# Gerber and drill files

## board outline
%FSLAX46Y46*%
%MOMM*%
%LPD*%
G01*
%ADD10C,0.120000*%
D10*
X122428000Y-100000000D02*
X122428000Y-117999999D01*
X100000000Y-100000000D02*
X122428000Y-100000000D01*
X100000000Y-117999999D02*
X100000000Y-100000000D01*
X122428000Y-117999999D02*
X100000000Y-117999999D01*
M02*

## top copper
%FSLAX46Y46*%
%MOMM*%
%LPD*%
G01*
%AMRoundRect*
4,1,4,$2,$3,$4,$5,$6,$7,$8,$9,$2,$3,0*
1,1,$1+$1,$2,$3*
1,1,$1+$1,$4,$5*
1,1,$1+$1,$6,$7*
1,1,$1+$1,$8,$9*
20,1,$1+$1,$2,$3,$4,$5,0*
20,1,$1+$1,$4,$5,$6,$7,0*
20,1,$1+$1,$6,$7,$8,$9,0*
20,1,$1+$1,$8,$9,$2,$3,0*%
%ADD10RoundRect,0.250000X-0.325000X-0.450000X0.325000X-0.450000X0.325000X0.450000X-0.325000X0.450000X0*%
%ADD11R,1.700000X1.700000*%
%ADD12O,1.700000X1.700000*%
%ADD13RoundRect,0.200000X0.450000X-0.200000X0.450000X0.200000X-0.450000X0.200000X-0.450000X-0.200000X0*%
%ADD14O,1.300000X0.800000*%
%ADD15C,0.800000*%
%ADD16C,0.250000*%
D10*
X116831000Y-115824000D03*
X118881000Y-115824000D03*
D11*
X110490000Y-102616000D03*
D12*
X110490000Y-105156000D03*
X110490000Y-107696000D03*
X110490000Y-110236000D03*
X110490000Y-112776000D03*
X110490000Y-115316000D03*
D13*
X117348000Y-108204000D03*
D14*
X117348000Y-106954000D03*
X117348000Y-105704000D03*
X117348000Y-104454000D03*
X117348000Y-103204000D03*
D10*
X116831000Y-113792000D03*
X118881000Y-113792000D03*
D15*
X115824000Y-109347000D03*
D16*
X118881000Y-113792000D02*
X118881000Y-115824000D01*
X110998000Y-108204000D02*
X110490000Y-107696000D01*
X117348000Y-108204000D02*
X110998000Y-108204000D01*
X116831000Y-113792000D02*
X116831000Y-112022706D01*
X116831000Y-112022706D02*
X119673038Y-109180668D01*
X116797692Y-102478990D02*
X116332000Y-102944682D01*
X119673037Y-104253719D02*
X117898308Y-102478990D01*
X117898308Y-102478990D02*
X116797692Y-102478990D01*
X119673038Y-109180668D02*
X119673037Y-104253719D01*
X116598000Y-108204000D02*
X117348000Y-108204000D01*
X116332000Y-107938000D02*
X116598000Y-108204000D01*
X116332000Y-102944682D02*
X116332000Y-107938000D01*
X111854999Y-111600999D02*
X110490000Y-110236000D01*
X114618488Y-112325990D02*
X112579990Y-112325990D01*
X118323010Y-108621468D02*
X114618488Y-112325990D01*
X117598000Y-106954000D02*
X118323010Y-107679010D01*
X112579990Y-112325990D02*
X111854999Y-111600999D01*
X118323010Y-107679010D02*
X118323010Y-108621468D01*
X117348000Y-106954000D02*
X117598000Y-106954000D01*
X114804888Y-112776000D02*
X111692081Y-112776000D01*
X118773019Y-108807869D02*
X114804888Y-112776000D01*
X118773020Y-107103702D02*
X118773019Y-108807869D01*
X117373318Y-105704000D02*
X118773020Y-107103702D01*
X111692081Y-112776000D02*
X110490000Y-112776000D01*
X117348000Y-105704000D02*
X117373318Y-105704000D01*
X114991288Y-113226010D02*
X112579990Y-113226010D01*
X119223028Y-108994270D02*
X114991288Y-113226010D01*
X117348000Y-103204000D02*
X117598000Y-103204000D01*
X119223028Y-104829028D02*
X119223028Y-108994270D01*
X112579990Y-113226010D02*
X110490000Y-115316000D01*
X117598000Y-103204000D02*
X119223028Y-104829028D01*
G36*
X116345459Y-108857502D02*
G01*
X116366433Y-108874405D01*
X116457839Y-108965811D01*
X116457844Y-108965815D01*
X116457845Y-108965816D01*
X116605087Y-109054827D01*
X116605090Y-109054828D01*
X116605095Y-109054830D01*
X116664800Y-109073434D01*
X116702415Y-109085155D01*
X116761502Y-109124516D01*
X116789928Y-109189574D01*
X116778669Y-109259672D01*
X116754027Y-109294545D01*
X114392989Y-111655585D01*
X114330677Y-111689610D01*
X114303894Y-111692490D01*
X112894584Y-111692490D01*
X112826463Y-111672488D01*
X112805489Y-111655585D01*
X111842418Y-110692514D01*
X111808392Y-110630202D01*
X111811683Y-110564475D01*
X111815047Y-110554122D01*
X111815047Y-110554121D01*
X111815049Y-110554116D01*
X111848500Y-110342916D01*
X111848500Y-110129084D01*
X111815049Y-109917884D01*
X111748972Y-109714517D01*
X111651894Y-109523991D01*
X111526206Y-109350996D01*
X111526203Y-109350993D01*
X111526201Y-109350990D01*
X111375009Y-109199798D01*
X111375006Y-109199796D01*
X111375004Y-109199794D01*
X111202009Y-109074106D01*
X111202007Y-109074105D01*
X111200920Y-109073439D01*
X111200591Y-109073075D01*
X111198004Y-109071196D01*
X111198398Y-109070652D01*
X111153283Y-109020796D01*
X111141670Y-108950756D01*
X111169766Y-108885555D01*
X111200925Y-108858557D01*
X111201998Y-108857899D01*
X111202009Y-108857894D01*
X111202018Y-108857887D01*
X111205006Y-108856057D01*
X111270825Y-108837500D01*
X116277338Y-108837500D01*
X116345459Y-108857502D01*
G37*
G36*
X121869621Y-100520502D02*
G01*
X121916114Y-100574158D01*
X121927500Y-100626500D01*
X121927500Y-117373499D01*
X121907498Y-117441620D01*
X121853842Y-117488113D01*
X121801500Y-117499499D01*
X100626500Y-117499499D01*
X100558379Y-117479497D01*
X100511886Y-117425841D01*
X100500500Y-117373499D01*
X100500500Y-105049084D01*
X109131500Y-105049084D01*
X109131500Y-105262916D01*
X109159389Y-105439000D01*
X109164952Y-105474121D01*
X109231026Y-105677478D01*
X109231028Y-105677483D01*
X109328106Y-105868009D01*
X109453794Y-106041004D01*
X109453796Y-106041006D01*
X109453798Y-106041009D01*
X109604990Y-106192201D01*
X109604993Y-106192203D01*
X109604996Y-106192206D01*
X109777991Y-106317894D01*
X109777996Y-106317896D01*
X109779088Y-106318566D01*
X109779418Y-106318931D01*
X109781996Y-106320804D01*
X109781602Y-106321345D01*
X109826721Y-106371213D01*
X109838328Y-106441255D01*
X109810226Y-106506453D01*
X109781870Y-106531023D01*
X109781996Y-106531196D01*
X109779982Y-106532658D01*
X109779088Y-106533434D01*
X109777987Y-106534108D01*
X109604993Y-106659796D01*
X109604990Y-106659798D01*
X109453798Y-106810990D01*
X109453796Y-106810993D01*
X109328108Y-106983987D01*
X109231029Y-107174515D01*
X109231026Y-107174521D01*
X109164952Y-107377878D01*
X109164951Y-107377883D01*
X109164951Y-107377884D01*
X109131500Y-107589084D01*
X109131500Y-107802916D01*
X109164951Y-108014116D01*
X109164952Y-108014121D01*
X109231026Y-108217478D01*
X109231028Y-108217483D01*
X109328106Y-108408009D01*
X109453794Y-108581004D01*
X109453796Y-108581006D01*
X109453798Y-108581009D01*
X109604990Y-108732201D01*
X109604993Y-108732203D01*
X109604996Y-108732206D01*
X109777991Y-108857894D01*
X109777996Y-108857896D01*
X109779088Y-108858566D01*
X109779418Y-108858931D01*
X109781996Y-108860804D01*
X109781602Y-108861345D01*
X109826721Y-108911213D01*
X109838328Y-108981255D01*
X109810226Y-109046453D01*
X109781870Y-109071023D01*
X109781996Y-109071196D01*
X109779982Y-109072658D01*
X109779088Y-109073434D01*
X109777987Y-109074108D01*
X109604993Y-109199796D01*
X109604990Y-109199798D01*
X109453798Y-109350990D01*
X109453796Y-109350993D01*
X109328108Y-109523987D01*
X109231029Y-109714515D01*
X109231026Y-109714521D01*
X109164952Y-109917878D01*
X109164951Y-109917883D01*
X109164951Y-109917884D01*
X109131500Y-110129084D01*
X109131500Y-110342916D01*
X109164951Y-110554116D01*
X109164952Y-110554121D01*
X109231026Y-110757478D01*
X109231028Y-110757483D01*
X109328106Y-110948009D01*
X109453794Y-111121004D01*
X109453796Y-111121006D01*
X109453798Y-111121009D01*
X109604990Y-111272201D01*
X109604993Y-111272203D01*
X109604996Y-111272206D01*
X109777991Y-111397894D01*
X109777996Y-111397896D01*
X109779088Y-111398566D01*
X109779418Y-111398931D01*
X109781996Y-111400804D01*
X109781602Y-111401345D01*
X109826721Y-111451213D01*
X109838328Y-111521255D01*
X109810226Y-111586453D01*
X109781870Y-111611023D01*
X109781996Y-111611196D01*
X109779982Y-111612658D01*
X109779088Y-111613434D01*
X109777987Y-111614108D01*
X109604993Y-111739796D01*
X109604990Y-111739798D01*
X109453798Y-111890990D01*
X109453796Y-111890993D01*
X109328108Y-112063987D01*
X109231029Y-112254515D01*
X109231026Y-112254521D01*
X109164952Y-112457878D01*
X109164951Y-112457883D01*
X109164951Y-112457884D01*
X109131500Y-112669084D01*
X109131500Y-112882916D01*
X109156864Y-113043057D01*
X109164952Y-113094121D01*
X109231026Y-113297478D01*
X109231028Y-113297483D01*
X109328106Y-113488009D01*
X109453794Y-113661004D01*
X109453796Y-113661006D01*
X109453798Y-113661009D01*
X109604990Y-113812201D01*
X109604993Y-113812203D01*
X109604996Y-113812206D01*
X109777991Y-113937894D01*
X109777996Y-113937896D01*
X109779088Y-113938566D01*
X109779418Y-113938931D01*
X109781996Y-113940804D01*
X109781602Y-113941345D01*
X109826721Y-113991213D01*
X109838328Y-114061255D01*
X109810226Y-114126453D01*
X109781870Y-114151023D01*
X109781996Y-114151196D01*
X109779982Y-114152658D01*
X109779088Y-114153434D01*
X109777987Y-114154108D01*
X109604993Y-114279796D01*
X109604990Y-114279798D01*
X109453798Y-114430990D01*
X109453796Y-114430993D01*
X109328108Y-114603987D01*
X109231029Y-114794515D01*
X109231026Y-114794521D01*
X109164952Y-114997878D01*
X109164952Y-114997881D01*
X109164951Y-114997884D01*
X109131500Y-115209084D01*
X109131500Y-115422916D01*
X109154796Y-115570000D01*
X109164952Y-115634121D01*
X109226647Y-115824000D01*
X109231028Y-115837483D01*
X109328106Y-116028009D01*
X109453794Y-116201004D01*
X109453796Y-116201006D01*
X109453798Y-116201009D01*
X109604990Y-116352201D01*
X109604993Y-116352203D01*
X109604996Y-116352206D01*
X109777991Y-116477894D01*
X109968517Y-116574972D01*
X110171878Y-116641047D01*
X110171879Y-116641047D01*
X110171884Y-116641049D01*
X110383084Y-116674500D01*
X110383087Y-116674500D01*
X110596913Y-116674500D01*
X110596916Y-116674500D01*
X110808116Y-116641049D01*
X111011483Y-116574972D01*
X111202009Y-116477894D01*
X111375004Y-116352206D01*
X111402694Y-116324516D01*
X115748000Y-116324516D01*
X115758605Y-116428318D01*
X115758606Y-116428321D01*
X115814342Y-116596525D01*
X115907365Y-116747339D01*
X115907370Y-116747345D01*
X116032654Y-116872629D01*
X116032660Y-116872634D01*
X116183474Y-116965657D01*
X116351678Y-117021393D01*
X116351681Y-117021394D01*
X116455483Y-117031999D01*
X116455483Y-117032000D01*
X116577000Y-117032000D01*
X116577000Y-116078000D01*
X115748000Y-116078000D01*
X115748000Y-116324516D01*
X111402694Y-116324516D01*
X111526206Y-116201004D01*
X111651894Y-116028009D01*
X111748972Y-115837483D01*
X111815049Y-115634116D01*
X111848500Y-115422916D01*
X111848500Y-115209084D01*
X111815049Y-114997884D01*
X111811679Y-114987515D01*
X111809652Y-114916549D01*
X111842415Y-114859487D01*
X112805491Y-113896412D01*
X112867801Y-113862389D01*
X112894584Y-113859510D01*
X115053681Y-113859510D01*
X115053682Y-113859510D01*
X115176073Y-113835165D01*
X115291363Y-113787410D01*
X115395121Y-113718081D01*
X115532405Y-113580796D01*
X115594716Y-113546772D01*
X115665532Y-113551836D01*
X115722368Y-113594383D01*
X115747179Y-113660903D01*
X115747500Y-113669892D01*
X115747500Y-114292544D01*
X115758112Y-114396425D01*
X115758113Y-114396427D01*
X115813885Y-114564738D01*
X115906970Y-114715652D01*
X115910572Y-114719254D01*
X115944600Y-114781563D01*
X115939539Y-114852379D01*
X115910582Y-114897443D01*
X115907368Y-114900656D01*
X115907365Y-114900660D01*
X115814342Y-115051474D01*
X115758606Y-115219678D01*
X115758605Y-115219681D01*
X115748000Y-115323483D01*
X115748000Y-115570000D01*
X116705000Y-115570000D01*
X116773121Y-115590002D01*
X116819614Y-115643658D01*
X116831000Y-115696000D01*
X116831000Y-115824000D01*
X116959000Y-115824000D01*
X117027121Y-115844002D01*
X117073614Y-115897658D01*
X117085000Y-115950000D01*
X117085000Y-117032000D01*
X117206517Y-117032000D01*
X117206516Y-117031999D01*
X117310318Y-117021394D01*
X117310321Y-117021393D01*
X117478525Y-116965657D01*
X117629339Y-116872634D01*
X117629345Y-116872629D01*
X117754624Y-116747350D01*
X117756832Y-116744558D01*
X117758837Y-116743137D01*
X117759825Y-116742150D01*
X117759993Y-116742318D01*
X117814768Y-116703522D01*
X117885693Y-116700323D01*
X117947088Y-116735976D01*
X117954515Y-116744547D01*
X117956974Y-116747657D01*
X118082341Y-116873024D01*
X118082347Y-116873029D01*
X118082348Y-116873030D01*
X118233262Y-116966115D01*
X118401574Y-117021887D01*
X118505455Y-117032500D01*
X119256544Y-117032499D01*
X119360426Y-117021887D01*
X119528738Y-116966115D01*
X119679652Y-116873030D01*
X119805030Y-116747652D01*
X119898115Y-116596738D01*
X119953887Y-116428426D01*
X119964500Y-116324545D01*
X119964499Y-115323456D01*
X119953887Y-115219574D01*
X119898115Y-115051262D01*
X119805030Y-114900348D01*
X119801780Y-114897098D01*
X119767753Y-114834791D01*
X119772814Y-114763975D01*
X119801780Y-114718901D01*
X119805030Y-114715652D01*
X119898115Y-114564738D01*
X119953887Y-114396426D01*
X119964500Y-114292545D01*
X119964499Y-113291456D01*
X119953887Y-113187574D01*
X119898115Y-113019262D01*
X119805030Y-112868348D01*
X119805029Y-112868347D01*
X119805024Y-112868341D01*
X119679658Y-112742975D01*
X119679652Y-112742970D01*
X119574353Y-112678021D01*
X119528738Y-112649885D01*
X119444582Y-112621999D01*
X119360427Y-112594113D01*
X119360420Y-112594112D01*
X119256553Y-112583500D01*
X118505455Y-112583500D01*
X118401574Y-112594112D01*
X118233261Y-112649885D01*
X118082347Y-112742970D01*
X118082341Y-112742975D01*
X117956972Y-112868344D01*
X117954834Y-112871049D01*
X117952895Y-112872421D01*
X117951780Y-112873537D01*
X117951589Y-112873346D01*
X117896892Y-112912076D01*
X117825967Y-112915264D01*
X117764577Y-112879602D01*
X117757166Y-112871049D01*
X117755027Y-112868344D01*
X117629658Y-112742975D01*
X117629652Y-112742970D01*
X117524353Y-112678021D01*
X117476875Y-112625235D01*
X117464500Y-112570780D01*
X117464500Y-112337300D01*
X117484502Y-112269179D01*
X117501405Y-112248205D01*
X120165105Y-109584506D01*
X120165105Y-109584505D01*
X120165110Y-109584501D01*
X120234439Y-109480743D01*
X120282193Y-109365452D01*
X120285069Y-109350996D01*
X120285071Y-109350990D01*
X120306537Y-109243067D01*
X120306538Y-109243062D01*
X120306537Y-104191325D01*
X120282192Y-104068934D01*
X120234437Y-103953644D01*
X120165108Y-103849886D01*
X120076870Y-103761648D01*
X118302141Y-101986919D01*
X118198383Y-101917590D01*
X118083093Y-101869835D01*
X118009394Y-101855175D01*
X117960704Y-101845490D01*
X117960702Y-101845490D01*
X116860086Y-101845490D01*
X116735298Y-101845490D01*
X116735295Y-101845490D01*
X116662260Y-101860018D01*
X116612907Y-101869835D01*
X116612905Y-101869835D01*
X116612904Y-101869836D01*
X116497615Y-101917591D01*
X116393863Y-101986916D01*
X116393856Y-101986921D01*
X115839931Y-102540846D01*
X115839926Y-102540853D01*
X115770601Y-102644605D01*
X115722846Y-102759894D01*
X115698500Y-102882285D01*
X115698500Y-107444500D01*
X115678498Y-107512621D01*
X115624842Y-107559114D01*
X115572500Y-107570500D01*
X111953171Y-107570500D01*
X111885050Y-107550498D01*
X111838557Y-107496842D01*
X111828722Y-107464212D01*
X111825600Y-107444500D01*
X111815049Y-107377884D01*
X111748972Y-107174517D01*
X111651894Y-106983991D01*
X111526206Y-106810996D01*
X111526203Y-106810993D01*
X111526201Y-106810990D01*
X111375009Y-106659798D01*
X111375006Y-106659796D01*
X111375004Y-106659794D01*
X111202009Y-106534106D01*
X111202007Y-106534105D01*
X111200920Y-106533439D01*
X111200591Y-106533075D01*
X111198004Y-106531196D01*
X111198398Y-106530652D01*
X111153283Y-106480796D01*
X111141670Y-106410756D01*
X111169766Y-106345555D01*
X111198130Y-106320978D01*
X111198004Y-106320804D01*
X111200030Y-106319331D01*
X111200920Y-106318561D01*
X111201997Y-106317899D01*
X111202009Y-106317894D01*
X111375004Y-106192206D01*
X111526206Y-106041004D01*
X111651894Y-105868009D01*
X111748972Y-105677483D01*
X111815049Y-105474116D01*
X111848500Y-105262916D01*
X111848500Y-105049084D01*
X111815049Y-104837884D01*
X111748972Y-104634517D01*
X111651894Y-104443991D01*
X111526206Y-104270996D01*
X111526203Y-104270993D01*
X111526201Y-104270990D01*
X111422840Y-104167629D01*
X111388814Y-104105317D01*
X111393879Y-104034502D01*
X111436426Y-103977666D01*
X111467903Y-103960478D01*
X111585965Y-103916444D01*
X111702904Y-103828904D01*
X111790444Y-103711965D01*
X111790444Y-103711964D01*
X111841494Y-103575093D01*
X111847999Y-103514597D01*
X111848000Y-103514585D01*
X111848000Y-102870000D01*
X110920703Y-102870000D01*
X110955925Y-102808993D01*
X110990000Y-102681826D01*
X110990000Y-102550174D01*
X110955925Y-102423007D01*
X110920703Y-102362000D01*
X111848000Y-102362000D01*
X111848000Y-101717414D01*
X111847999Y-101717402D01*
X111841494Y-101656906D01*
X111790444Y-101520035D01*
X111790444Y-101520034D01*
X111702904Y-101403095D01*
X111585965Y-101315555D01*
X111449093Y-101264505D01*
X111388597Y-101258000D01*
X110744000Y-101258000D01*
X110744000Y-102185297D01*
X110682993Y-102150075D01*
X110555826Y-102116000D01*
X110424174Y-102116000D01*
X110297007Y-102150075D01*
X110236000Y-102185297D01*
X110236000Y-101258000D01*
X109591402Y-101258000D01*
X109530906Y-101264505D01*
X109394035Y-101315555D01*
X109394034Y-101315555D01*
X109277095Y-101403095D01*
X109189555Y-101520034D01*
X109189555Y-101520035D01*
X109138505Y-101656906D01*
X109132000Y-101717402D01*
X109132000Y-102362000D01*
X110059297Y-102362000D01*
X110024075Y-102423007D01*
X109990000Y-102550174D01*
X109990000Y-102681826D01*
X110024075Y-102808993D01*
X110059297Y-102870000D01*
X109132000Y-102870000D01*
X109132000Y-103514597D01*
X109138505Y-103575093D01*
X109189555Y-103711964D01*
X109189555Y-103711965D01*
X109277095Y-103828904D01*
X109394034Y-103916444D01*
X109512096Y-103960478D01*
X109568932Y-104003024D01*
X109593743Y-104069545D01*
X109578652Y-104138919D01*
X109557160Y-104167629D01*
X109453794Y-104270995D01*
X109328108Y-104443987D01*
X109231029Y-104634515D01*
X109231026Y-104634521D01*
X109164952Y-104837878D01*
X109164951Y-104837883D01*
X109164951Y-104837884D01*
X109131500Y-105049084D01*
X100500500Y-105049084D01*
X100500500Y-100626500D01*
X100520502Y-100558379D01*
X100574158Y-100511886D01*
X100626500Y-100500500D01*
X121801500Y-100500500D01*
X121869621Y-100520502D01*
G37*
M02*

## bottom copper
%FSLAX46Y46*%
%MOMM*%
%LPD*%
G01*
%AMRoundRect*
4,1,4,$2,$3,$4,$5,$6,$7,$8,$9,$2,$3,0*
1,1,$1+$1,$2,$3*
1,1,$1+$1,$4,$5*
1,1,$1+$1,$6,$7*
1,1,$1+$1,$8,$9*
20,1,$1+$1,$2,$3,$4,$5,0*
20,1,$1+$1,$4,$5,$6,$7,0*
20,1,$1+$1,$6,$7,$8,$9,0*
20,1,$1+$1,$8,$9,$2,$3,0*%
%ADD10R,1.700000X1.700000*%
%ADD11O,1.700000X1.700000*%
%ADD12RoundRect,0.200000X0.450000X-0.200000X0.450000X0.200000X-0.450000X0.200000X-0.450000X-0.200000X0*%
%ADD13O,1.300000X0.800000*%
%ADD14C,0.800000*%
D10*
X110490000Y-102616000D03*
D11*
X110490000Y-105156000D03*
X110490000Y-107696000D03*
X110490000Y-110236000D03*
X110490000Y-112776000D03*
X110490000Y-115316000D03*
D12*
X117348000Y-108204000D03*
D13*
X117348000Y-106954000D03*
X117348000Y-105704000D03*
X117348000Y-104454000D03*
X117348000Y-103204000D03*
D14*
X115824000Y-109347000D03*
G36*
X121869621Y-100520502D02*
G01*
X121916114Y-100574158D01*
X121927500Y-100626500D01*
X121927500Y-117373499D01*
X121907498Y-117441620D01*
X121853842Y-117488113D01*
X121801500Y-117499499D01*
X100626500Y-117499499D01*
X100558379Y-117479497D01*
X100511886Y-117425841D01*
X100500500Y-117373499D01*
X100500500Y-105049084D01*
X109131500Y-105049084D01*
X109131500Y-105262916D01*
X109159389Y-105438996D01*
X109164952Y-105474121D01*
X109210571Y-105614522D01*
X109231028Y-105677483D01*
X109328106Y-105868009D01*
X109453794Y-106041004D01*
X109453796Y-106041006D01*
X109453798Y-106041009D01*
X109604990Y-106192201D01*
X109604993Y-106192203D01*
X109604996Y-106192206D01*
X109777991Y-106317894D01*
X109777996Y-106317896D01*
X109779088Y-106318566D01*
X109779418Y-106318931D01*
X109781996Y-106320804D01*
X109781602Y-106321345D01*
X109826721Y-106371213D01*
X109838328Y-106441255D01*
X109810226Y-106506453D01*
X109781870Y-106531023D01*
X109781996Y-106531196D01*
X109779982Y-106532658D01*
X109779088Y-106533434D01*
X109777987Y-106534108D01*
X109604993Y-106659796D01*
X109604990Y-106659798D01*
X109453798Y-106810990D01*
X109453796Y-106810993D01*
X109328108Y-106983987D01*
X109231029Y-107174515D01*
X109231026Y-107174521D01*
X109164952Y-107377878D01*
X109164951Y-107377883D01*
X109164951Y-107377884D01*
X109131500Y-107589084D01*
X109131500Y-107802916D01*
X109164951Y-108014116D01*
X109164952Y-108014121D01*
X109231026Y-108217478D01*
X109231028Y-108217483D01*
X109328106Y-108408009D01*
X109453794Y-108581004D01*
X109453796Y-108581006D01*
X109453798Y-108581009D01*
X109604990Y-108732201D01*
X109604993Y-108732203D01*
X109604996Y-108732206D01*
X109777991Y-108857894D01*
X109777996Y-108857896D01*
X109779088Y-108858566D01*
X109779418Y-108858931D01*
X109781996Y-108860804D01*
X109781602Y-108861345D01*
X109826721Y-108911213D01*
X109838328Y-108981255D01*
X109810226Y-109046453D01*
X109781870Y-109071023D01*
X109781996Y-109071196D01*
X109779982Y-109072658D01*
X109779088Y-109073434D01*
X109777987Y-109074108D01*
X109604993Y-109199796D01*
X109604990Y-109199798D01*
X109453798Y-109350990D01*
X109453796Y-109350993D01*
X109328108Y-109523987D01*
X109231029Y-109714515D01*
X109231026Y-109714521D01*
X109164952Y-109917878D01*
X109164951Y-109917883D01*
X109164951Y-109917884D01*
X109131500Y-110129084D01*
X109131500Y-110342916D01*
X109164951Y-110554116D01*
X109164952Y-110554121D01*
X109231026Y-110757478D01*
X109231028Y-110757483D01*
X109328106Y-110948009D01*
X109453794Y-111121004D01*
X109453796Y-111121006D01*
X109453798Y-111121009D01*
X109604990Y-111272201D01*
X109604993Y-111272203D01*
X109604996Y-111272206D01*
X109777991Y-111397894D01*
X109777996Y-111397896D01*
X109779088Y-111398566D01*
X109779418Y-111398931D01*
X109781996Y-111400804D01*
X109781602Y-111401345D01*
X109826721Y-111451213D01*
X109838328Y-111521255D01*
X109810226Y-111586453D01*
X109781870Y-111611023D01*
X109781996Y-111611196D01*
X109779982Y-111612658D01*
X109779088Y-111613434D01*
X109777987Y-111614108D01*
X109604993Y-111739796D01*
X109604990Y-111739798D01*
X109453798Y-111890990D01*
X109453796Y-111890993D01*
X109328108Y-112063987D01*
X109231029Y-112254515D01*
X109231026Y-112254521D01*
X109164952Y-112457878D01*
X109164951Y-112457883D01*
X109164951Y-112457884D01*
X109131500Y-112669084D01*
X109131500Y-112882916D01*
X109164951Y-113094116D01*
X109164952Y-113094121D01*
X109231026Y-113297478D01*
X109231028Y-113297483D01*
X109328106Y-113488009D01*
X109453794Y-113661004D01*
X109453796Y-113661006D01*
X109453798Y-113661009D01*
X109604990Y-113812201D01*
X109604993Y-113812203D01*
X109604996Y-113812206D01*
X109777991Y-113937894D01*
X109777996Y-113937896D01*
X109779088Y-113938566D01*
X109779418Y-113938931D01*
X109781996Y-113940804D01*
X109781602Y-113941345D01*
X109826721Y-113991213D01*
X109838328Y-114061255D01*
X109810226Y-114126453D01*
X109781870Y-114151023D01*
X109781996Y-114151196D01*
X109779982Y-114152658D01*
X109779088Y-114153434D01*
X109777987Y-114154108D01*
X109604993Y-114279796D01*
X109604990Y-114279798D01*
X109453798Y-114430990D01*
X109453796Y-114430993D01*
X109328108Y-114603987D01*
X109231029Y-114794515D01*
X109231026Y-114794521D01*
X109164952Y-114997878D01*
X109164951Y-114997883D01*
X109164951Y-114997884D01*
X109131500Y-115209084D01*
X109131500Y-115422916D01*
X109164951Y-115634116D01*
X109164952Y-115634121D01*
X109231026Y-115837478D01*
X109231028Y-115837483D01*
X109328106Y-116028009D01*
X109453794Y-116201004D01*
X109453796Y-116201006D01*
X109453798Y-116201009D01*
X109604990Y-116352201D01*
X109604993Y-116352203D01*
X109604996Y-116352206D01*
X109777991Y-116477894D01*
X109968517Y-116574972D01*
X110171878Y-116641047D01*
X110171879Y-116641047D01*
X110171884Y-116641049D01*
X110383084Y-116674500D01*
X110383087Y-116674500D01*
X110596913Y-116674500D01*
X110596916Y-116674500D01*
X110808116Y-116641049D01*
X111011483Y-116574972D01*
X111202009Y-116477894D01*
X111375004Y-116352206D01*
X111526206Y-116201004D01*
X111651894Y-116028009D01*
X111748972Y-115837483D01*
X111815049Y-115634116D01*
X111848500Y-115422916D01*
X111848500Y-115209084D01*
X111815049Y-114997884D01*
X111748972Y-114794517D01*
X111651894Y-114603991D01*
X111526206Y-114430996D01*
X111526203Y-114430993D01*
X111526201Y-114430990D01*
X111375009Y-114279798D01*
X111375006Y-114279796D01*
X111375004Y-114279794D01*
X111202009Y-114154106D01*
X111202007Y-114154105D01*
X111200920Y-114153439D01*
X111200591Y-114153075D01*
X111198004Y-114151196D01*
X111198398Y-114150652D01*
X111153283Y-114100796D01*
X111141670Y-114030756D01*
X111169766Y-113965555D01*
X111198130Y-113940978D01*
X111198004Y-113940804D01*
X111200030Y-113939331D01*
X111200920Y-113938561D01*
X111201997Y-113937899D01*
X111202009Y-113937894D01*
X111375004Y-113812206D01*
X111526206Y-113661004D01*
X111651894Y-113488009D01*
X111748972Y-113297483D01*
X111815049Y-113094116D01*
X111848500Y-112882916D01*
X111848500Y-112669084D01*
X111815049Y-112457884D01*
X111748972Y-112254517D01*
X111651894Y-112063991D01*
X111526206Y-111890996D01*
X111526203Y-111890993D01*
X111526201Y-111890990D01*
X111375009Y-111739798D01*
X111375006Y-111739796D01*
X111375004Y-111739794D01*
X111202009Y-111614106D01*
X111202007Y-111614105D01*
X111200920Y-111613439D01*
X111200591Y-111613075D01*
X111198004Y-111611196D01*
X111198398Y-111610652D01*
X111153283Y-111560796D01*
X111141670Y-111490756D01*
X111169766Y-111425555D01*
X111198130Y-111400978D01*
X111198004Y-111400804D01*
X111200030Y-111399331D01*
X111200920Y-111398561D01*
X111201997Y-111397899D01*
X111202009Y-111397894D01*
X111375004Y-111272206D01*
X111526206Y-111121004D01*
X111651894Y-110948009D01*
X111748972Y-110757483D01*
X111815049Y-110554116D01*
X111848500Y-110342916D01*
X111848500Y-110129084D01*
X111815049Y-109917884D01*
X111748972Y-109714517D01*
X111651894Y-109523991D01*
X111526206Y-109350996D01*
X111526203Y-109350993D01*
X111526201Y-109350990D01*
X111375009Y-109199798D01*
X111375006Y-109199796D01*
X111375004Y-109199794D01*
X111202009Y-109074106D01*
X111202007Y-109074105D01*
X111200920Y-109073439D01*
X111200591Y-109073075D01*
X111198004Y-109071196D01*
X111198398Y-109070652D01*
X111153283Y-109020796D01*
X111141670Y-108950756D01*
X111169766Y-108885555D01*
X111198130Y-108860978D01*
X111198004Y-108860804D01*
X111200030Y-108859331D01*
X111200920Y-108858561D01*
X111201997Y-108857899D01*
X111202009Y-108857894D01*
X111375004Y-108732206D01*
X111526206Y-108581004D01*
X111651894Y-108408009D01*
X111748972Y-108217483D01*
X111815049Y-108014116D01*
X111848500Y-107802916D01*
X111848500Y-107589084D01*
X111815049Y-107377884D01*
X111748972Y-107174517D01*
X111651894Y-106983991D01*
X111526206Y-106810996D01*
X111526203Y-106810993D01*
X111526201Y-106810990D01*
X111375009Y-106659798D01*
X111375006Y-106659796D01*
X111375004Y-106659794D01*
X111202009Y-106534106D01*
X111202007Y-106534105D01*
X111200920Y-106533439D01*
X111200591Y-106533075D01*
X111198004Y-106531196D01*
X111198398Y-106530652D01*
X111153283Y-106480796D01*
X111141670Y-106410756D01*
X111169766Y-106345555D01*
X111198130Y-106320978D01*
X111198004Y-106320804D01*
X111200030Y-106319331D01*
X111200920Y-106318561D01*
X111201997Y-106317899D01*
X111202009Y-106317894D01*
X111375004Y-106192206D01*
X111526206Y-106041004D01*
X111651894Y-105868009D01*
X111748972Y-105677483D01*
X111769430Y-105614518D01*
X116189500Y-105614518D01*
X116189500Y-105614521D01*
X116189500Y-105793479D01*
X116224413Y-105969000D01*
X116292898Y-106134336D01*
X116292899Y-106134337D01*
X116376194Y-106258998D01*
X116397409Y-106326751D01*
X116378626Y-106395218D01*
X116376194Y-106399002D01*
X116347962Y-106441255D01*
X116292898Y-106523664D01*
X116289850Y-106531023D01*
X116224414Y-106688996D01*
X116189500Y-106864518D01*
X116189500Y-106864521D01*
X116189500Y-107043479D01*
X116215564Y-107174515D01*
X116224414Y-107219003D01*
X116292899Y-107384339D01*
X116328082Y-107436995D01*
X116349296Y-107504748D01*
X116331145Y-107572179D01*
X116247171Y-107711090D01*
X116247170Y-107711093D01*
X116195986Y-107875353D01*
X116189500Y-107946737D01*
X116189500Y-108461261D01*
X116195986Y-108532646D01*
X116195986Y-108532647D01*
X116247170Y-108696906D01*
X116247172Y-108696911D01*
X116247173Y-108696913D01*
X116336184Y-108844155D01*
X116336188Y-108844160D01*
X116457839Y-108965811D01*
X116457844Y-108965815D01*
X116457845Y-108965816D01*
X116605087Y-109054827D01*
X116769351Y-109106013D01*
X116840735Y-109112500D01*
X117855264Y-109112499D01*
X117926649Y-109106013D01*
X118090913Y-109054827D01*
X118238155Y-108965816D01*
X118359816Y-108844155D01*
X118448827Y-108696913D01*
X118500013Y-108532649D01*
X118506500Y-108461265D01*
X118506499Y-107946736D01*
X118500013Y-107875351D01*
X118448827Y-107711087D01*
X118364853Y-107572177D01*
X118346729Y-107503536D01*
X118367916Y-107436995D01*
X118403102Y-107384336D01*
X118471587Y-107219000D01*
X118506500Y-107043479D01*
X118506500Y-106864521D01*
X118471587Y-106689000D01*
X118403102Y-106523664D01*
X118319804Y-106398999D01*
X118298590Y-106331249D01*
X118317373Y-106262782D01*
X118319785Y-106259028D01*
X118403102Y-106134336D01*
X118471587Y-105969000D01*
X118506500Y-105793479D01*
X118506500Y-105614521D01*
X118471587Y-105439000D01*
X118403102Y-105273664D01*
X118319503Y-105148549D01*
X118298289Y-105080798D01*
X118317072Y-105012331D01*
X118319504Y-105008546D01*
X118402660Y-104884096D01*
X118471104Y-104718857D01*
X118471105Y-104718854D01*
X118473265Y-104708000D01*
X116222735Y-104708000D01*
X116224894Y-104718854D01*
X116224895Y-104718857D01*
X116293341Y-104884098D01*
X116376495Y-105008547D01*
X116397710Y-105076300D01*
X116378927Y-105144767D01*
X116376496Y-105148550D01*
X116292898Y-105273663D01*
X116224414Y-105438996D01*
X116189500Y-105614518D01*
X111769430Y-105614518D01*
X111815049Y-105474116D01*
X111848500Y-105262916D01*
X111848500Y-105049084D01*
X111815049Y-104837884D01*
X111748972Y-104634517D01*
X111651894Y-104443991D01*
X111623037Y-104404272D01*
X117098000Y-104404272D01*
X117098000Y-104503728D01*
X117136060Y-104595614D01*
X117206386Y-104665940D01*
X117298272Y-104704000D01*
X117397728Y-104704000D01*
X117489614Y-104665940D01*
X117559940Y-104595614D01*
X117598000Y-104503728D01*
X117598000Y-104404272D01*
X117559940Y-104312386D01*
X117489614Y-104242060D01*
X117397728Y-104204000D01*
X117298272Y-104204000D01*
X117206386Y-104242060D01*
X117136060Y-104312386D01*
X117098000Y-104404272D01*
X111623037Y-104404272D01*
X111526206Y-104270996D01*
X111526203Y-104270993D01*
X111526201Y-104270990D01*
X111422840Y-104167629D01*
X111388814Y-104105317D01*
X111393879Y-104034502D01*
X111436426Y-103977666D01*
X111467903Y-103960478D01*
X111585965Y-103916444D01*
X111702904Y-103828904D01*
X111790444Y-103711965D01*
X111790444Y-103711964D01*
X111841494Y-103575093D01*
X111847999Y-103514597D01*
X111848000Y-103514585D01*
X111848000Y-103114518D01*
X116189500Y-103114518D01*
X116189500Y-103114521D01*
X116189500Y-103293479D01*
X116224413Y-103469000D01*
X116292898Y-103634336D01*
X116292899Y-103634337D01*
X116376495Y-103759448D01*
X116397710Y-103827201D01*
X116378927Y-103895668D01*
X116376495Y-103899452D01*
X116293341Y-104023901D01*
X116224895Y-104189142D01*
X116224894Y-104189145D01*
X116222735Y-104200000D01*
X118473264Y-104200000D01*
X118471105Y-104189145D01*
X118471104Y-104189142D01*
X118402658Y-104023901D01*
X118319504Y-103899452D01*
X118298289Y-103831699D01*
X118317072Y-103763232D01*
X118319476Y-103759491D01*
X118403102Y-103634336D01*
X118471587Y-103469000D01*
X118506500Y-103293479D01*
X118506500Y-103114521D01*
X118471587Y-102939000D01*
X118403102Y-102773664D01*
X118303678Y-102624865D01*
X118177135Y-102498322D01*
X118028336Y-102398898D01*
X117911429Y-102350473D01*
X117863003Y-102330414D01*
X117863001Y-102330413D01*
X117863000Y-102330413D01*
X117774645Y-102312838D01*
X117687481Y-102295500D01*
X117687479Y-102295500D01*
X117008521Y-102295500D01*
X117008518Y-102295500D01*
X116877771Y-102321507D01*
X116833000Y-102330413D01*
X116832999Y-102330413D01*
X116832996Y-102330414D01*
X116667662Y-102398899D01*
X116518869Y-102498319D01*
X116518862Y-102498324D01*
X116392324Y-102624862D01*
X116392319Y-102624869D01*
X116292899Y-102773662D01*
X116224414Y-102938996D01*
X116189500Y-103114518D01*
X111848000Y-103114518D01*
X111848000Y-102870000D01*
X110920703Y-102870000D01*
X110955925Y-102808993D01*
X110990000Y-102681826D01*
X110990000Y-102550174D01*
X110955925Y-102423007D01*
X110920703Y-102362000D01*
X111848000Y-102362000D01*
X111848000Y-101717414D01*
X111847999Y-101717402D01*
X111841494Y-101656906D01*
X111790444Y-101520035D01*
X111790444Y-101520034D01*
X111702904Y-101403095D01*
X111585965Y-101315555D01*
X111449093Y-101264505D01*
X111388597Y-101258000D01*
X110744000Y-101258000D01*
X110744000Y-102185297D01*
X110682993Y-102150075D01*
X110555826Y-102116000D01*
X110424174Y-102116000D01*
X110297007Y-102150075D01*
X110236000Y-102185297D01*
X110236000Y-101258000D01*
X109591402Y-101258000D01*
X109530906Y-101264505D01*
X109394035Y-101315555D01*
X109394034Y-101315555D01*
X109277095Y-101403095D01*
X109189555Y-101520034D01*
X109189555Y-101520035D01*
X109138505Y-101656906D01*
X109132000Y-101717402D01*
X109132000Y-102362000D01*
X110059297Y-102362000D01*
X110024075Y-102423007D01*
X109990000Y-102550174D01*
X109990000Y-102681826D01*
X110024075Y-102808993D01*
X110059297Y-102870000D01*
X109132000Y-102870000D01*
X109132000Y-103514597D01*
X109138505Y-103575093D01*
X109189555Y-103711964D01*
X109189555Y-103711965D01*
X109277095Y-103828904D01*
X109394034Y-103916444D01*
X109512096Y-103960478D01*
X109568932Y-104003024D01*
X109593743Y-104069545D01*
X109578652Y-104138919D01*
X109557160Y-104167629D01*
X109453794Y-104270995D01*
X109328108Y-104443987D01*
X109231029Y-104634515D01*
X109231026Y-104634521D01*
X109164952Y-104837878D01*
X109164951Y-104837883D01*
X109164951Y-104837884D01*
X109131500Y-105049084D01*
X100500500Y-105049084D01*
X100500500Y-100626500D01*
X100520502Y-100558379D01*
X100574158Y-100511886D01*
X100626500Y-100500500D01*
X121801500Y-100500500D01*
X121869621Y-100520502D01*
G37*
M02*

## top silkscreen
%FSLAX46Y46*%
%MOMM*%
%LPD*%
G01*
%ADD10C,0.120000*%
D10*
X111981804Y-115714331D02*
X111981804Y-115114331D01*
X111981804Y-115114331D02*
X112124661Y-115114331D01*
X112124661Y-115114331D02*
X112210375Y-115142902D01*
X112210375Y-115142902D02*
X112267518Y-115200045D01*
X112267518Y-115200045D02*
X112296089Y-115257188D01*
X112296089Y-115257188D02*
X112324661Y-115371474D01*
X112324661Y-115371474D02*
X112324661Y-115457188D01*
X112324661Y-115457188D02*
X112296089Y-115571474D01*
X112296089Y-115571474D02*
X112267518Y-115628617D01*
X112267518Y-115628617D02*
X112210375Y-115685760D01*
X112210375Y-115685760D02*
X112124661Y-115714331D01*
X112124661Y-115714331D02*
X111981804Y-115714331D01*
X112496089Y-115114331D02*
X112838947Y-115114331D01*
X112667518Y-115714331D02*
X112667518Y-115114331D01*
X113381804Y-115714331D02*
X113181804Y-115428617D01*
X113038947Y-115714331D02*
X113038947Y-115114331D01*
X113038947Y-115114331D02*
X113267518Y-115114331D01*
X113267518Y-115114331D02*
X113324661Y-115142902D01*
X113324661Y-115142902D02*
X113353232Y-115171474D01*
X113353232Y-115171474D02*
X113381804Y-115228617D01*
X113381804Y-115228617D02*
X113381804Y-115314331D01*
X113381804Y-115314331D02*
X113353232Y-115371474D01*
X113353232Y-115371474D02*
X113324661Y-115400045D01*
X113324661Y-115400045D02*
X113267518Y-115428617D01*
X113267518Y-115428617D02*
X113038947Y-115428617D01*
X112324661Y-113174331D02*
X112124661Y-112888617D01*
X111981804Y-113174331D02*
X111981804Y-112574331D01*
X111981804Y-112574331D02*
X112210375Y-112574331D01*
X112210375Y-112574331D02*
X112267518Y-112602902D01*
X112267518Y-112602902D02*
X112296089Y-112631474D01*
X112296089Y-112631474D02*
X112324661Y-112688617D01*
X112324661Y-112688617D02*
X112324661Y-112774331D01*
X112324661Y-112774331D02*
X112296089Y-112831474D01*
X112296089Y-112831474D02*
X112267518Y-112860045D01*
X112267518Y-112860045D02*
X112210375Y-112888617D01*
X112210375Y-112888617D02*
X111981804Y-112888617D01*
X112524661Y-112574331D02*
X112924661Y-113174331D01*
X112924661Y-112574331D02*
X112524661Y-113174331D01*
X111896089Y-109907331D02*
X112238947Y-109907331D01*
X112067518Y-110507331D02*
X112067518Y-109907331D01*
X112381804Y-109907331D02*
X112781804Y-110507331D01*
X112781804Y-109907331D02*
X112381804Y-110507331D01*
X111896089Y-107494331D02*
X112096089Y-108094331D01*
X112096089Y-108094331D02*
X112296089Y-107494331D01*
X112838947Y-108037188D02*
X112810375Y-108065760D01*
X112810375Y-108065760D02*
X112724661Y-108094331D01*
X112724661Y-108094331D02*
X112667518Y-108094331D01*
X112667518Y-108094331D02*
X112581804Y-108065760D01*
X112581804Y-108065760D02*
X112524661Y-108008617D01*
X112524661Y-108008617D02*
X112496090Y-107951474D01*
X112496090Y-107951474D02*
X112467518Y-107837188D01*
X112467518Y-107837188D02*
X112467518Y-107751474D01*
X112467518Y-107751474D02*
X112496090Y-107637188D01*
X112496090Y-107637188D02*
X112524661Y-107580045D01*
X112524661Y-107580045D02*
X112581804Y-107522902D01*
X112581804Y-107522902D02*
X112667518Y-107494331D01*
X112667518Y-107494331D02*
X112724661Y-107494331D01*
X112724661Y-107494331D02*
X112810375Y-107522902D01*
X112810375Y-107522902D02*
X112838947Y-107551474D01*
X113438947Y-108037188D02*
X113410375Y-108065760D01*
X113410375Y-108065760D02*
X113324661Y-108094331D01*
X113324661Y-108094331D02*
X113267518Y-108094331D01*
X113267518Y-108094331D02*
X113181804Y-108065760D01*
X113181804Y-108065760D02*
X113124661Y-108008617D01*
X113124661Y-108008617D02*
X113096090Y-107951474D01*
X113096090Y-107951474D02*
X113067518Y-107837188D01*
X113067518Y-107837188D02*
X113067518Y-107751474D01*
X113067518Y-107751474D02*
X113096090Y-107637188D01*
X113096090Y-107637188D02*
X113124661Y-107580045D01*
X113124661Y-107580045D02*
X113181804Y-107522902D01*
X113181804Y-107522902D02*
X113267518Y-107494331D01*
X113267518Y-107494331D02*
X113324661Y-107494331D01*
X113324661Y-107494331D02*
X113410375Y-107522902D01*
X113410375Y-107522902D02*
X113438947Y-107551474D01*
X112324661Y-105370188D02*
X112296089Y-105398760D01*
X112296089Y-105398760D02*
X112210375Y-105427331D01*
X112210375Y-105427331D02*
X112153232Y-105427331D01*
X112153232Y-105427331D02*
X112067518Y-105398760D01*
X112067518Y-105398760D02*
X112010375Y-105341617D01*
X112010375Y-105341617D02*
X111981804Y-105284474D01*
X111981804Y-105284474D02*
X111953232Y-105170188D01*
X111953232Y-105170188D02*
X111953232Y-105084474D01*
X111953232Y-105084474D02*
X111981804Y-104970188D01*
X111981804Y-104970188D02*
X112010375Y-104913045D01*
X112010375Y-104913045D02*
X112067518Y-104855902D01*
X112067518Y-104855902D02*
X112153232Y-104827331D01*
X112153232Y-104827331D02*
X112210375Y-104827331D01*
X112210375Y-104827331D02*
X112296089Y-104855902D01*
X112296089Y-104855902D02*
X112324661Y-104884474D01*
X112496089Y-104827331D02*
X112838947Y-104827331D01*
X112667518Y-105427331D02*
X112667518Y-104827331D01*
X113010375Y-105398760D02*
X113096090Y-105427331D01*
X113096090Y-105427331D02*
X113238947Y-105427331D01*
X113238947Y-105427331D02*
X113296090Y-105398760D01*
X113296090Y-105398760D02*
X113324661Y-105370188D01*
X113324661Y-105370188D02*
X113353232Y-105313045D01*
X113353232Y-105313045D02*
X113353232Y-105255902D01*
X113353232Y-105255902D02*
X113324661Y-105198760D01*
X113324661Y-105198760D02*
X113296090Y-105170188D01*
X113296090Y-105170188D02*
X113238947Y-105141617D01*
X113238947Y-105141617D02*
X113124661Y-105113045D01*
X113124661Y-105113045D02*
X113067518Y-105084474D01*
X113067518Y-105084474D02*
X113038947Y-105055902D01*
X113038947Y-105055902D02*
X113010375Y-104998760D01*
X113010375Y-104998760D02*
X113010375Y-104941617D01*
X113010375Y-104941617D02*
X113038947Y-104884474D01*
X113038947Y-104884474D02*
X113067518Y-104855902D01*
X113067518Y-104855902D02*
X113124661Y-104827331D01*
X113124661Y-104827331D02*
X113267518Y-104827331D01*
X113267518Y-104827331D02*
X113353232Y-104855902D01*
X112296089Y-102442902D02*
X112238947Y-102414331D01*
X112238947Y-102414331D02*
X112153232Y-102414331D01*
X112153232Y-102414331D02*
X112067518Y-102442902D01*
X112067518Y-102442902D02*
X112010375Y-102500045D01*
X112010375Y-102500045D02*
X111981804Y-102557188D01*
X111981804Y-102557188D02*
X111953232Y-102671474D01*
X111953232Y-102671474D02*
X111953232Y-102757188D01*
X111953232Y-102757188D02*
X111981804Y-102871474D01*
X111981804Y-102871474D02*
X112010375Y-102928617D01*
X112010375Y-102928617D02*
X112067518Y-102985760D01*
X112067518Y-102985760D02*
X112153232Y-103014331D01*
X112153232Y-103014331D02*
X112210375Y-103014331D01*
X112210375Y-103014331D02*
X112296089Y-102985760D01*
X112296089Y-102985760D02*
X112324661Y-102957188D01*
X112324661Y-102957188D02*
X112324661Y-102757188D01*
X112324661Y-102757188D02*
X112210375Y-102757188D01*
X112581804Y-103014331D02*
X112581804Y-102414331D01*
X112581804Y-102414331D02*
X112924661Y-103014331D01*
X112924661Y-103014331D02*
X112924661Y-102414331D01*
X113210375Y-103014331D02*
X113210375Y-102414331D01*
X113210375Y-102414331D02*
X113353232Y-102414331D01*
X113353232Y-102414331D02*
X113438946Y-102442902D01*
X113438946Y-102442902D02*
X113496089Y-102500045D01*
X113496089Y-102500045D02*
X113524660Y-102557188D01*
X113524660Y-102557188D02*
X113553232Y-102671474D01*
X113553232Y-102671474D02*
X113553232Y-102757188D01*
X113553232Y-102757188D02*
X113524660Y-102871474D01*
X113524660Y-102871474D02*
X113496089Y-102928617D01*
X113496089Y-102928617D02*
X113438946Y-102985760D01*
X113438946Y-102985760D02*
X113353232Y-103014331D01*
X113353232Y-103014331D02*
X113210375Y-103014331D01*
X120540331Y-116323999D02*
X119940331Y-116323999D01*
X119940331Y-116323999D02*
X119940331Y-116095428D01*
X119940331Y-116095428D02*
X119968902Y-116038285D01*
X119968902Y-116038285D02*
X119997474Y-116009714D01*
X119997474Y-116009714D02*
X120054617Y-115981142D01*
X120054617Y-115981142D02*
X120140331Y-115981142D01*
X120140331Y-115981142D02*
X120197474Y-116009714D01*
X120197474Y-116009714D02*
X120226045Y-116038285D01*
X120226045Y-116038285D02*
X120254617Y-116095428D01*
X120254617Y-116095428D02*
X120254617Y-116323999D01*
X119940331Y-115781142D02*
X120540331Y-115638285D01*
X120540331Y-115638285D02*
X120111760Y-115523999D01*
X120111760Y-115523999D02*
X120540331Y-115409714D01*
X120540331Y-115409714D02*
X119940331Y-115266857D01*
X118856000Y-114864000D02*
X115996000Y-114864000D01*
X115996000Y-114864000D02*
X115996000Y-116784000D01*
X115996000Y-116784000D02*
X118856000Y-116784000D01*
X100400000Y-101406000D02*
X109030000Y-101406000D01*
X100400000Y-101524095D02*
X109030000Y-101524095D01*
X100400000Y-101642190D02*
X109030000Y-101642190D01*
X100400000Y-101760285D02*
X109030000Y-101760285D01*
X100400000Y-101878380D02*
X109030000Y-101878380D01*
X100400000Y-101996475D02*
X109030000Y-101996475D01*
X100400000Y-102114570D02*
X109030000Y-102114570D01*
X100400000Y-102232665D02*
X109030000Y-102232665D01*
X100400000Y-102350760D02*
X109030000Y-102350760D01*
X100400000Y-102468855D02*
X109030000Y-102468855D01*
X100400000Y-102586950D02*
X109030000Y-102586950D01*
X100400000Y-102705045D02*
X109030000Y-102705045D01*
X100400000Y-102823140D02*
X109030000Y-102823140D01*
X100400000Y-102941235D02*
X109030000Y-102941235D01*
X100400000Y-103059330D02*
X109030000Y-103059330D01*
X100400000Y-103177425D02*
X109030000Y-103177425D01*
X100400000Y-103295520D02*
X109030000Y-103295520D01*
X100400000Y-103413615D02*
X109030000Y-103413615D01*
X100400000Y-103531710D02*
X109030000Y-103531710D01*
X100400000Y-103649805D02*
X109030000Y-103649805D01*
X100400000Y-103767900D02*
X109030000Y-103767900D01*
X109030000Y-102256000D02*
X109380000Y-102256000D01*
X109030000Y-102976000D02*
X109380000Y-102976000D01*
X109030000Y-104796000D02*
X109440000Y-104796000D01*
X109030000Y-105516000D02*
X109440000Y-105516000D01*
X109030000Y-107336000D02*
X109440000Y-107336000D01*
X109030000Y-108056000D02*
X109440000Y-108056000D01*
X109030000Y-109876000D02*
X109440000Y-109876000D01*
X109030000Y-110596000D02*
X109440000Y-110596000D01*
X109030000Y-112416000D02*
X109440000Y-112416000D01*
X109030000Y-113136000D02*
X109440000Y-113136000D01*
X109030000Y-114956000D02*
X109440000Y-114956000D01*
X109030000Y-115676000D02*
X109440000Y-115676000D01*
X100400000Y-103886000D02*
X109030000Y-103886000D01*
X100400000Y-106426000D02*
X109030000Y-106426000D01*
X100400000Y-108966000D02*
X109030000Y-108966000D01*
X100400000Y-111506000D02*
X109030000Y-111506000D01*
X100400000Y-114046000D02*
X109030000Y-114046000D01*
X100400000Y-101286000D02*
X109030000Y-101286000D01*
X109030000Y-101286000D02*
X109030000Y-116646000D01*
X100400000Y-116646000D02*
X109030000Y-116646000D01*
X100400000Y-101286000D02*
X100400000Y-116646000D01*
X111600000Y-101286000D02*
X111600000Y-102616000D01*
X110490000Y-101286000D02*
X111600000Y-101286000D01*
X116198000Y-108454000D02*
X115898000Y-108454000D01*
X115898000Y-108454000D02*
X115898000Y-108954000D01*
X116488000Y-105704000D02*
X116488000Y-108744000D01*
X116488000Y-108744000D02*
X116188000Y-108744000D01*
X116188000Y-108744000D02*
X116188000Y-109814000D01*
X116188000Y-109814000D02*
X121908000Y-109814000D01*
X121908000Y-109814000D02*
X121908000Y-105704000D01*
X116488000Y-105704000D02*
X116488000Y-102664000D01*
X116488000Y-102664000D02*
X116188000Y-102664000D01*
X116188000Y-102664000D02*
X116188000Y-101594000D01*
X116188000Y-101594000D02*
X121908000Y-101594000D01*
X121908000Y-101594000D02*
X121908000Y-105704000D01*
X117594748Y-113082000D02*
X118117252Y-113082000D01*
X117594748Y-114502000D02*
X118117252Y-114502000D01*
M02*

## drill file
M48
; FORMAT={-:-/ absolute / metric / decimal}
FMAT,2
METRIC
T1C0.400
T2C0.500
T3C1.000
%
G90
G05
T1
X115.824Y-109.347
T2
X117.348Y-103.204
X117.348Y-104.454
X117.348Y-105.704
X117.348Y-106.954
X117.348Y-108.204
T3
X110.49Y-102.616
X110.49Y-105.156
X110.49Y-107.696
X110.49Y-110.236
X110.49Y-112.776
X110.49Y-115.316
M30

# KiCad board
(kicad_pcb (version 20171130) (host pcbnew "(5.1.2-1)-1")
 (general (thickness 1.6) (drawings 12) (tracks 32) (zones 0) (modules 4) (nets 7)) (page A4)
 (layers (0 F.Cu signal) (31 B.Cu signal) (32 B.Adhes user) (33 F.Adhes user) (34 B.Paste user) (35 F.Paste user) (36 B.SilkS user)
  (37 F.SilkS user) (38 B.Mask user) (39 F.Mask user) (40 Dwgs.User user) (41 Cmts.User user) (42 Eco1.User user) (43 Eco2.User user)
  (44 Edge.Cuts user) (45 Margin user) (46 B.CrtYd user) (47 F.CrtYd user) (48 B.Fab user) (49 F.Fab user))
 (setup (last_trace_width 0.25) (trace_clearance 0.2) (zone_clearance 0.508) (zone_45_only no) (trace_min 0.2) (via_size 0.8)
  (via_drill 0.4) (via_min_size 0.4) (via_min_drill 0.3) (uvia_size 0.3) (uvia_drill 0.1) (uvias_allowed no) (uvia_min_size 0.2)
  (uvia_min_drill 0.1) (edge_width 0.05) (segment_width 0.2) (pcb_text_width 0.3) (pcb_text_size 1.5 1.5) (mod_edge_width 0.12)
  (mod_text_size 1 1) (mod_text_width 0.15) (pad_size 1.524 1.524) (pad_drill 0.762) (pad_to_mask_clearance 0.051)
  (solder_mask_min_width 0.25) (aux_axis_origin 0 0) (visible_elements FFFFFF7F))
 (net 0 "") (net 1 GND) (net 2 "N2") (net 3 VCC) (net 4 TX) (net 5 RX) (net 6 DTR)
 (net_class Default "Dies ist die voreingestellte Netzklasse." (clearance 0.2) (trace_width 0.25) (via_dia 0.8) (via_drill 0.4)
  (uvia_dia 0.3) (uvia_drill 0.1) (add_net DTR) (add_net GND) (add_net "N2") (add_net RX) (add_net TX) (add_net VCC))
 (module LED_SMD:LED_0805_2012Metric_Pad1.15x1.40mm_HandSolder (layer F.Cu) (at 117.856 115.824)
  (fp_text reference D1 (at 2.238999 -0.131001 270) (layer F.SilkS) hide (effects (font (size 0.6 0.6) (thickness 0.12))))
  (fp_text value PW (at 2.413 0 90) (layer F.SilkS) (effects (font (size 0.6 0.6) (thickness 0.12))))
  (fp_line (start 1 -0.96) (end -1.86 -0.96) (layer F.SilkS) (width 0.12))
  (fp_line (start -1.86 -0.96) (end -1.86 0.96) (layer F.SilkS) (width 0.12))
  (fp_line (start -1.86 0.96) (end 1 0.96) (layer F.SilkS) (width 0.12))
  (pad 1 smd roundrect (at -1.025 0) (size 1.15 1.4) (layers F.Cu F.Paste F.Mask) (roundrect_rratio 0.217391) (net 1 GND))
  (pad 2 smd roundrect (at 1.025 0) (size 1.15 1.4) (layers F.Cu F.Paste F.Mask) (roundrect_rratio 0.217391) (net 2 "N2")))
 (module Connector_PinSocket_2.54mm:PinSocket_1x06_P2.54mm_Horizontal (layer F.Cu) (at 110.49 102.616)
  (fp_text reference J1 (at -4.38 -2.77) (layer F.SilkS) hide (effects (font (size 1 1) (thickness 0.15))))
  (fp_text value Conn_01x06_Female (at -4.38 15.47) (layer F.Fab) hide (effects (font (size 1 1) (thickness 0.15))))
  (fp_line (start -10.09 -1.21) (end -1.46 -1.21) (layer F.SilkS) (width 0.12))
  (fp_line (start -10.09 -1.091905) (end -1.46 -1.091905) (layer F.SilkS) (width 0.12))
  (fp_line (start -10.09 -0.97381) (end -1.46 -0.97381) (layer F.SilkS) (width 0.12))
  (fp_line (start -10.09 -0.855715) (end -1.46 -0.855715) (layer F.SilkS) (width 0.12))
  (fp_line (start -10.09 -0.73762) (end -1.46 -0.73762) (layer F.SilkS) (width 0.12))
  (fp_line (start -10.09 -0.619525) (end -1.46 -0.619525) (layer F.SilkS) (width 0.12))
  (fp_line (start -10.09 -0.50143) (end -1.46 -0.50143) (layer F.SilkS) (width 0.12))
  (fp_line (start -10.09 -0.383335) (end -1.46 -0.383335) (layer F.SilkS) (width 0.12))
  (fp_line (start -10.09 -0.26524) (end -1.46 -0.26524) (layer F.SilkS) (width 0.12))
  (fp_line (start -10.09 -0.147145) (end -1.46 -0.147145) (layer F.SilkS) (width 0.12))
  (fp_line (start -10.09 -0.02905) (end -1.46 -0.02905) (layer F.SilkS) (width 0.12))
  (fp_line (start -10.09 0.089045) (end -1.46 0.089045) (layer F.SilkS) (width 0.12))
  (fp_line (start -10.09 0.20714) (end -1.46 0.20714) (layer F.SilkS) (width 0.12))
  (fp_line (start -10.09 0.325235) (end -1.46 0.325235) (layer F.SilkS) (width 0.12))
  (fp_line (start -10.09 0.44333) (end -1.46 0.44333) (layer F.SilkS) (width 0.12))
  (fp_line (start -10.09 0.561425) (end -1.46 0.561425) (layer F.SilkS) (width 0.12))
  (fp_line (start -10.09 0.67952) (end -1.46 0.67952) (layer F.SilkS) (width 0.12))
  (fp_line (start -10.09 0.797615) (end -1.46 0.797615) (layer F.SilkS) (width 0.12))
  (fp_line (start -10.09 0.91571) (end -1.46 0.91571) (layer F.SilkS) (width 0.12))
  (fp_line (start -10.09 1.033805) (end -1.46 1.033805) (layer F.SilkS) (width 0.12))
  (fp_line (start -10.09 1.1519) (end -1.46 1.1519) (layer F.SilkS) (width 0.12))
  (fp_line (start -1.46 -0.36) (end -1.11 -0.36) (layer F.SilkS) (width 0.12))
  (fp_line (start -1.46 0.36) (end -1.11 0.36) (layer F.SilkS) (width 0.12))
  (fp_line (start -1.46 2.18) (end -1.05 2.18) (layer F.SilkS) (width 0.12))
  (fp_line (start -1.46 2.9) (end -1.05 2.9) (layer F.SilkS) (width 0.12))
  (fp_line (start -1.46 4.72) (end -1.05 4.72) (layer F.SilkS) (width 0.12))
  (fp_line (start -1.46 5.44) (end -1.05 5.44) (layer F.SilkS) (width 0.12))
  (fp_line (start -1.46 7.26) (end -1.05 7.26) (layer F.SilkS) (width 0.12))
  (fp_line (start -1.46 7.98) (end -1.05 7.98) (layer F.SilkS) (width 0.12))
  (fp_line (start -1.46 9.8) (end -1.05 9.8) (layer F.SilkS) (width 0.12))
  (fp_line (start -1.46 10.52) (end -1.05 10.52) (layer F.SilkS) (width 0.12))
  (fp_line (start -1.46 12.34) (end -1.05 12.34) (layer F.SilkS) (width 0.12))
  (fp_line (start -1.46 13.06) (end -1.05 13.06) (layer F.SilkS) (width 0.12))
  (fp_line (start -10.09 1.27) (end -1.46 1.27) (layer F.SilkS) (width 0.12))
  (fp_line (start -10.09 3.81) (end -1.46 3.81) (layer F.SilkS) (width 0.12))
  (fp_line (start -10.09 6.35) (end -1.46 6.35) (layer F.SilkS) (width 0.12))
  (fp_line (start -10.09 8.89) (end -1.46 8.89) (layer F.SilkS) (width 0.12))
  (fp_line (start -10.09 11.43) (end -1.46 11.43) (layer F.SilkS) (width 0.12))
  (fp_line (start -10.09 -1.33) (end -1.46 -1.33) (layer F.SilkS) (width 0.12))
  (fp_line (start -1.46 -1.33) (end -1.46 14.03) (layer F.SilkS) (width 0.12))
  (fp_line (start -10.09 14.03) (end -1.46 14.03) (layer F.SilkS) (width 0.12))
  (fp_line (start -10.09 -1.33) (end -10.09 14.03) (layer F.SilkS) (width 0.12))
  (fp_line (start 1.11 -1.33) (end 1.11 0) (layer F.SilkS) (width 0.12))
  (fp_line (start 0 -1.33) (end 1.11 -1.33) (layer F.SilkS) (width 0.12))
  (pad 1 thru_hole rect (at 0 0) (size 1.7 1.7) (drill 1) (layers *.Cu *.Mask) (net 1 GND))
  (pad 2 thru_hole oval (at 0 2.54) (size 1.7 1.7) (drill 1) (layers *.Cu *.Mask))
  (pad 3 thru_hole oval (at 0 5.08) (size 1.7 1.7) (drill 1) (layers *.Cu *.Mask) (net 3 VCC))
  (pad 4 thru_hole oval (at 0 7.62) (size 1.7 1.7) (drill 1) (layers *.Cu *.Mask) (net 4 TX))
  (pad 5 thru_hole oval (at 0 10.16) (size 1.7 1.7) (drill 1) (layers *.Cu *.Mask) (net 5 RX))
  (pad 6 thru_hole oval (at 0 12.7) (size 1.7 1.7) (drill 1) (layers *.Cu *.Mask) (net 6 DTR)))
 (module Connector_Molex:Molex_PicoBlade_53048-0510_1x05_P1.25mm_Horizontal (layer F.Cu) (at 117.348 108.204 90)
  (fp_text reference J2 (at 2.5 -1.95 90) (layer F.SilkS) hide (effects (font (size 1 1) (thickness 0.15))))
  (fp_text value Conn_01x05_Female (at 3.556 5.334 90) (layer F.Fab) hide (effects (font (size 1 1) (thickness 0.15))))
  (fp_line (start -0.25 -1.15) (end -0.25 -1.45) (layer F.SilkS) (width 0.12))
  (fp_line (start -0.25 -1.45) (end -0.75 -1.45) (layer F.SilkS) (width 0.12))
  (fp_line (start 2.5 -0.86) (end -0.54 -0.86) (layer F.SilkS) (width 0.12))
  (fp_line (start -0.54 -0.86) (end -0.54 -1.16) (layer F.SilkS) (width 0.12))
  (fp_line (start -0.54 -1.16) (end -1.61 -1.16) (layer F.SilkS) (width 0.12))
  (fp_line (start -1.61 -1.16) (end -1.61 4.56) (layer F.SilkS) (width 0.12))
  (fp_line (start -1.61 4.56) (end 2.5 4.56) (layer F.SilkS) (width 0.12))
  (fp_line (start 2.5 -0.86) (end 5.54 -0.86) (layer F.SilkS) (width 0.12))
  (fp_line (start 5.54 -0.86) (end 5.54 -1.16) (layer F.SilkS) (width 0.12))
  (fp_line (start 5.54 -1.16) (end 6.61 -1.16) (layer F.SilkS) (width 0.12))
  (fp_line (start 6.61 -1.16) (end 6.61 4.56) (layer F.SilkS) (width 0.12))
  (fp_line (start 6.61 4.56) (end 2.5 4.56) (layer F.SilkS) (width 0.12))
  (pad 1 thru_hole roundrect (at 0 0 90) (size 0.8 1.3) (drill 0.5) (layers *.Cu *.Mask) (roundrect_rratio 0.25) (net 3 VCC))
  (pad 2 thru_hole oval (at 1.25 0 90) (size 0.8 1.3) (drill 0.5) (layers *.Cu *.Mask) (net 4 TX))
  (pad 3 thru_hole oval (at 2.5 0 90) (size 0.8 1.3) (drill 0.5) (layers *.Cu *.Mask) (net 5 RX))
  (pad 4 thru_hole oval (at 3.75 0 90) (size 0.8 1.3) (drill 0.5) (layers *.Cu *.Mask) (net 1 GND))
  (pad 5 thru_hole oval (at 5 0 90) (size 0.8 1.3) (drill 0.5) (layers *.Cu *.Mask) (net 6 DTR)))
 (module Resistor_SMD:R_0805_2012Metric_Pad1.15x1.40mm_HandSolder (layer F.Cu) (at 117.856 113.792)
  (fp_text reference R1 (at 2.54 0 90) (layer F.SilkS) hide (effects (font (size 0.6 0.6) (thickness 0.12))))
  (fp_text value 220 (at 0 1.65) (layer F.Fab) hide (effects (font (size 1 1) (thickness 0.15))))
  (fp_line (start -0.261252 -0.71) (end 0.261252 -0.71) (layer F.SilkS) (width 0.12))
  (fp_line (start -0.261252 0.71) (end 0.261252 0.71) (layer F.SilkS) (width 0.12))
  (pad 1 smd roundrect (at -1.025 0) (size 1.15 1.4) (layers F.Cu F.Paste F.Mask) (roundrect_rratio 0.217391) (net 3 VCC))
  (pad 2 smd roundrect (at 1.025 0) (size 1.15 1.4) (layers F.Cu F.Paste F.Mask) (roundrect_rratio 0.217391) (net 2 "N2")))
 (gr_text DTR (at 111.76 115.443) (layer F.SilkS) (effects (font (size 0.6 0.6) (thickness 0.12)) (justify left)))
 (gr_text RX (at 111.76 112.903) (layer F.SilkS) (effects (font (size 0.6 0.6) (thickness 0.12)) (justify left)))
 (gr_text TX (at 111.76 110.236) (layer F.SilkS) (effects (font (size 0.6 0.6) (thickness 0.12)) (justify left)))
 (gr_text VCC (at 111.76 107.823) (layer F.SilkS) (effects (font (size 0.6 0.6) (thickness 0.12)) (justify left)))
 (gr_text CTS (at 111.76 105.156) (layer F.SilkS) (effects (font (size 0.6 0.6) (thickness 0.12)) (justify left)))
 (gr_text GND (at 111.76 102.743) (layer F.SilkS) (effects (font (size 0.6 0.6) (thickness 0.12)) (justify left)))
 (gr_line (start 122.428 100) (end 122.428 117.999999) (layer Edge.Cuts) (width 0.12))
 (gr_line (start 100 100) (end 122.428 100) (layer Edge.Cuts) (width 0.12))
 (gr_line (start 100 117.999999) (end 100 100) (layer Edge.Cuts) (width 0.12))
 (gr_line (start 122.428 117.999999) (end 100 117.999999) (layer Edge.Cuts) (width 0.12))
 (via (at 115.824 109.347) (size 0.8) (drill 0.4) (layers F.Cu B.Cu) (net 1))
 (segment (start 118.881 113.792) (end 118.881 115.824) (width 0.25) (layer F.Cu) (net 2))
 (segment (start 110.998 108.204) (end 110.49 107.696) (width 0.25) (layer F.Cu) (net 3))
 (segment (start 117.348 108.204) (end 110.998 108.204) (width 0.25) (layer F.Cu) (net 3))
 (segment (start 116.831 113.792) (end 116.831 112.022706) (width 0.25) (layer F.Cu) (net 3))
 (segment (start 116.831 112.022706) (end 119.673038 109.180668) (width 0.25) (layer F.Cu) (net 3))
 (segment (start 116.797692 102.47899) (end 116.332 102.944682) (width 0.25) (layer F.Cu) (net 3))
 (segment (start 119.673037 104.253719) (end 117.898308 102.47899) (width 0.25) (layer F.Cu) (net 3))
 (segment (start 117.898308 102.47899) (end 116.797692 102.47899) (width 0.25) (layer F.Cu) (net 3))
 (segment (start 119.673038 109.180668) (end 119.673037 104.253719) (width 0.25) (layer F.Cu) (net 3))
 (segment (start 116.598 108.204) (end 117.348 108.204) (width 0.25) (layer F.Cu) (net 3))
 (segment (start 116.332 107.938) (end 116.598 108.204) (width 0.25) (layer F.Cu) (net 3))
 (segment (start 116.332 102.944682) (end 116.332 107.938) (width 0.25) (layer F.Cu) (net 3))
 (segment (start 111.854999 111.600999) (end 110.49 110.236) (width 0.25) (layer F.Cu) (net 4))
 (segment (start 114.618488 112.32599) (end 112.57999 112.32599) (width 0.25) (layer F.Cu) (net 4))
 (segment (start 118.32301 108.621468) (end 114.618488 112.32599) (width 0.25) (layer F.Cu) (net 4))
 (segment (start 117.598 106.954) (end 118.32301 107.67901) (width 0.25) (layer F.Cu) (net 4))
 (segment (start 112.57999 112.32599) (end 111.854999 111.600999) (width 0.25) (layer F.Cu) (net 4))
 (segment (start 118.32301 107.67901) (end 118.32301 108.621468) (width 0.25) (layer F.Cu) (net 4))
 (segment (start 117.348 106.954) (end 117.598 106.954) (width 0.25) (layer F.Cu) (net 4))
 (segment (start 114.804888 112.776) (end 111.692081 112.776) (width 0.25) (layer F.Cu) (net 5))
 (segment (start 118.773019 108.807869) (end 114.804888 112.776) (width 0.25) (layer F.Cu) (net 5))
 (segment (start 118.77302 107.103702) (end 118.773019 108.807869) (width 0.25) (layer F.Cu) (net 5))
 (segment (start 117.373318 105.704) (end 118.77302 107.103702) (width 0.25) (layer F.Cu) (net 5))
 (segment (start 111.692081 112.776) (end 110.49 112.776) (width 0.25) (layer F.Cu) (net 5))
 (segment (start 117.348 105.704) (end 117.373318 105.704) (width 0.25) (layer F.Cu) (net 5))
 (segment (start 114.991288 113.22601) (end 112.57999 113.22601) (width 0.25) (layer F.Cu) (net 6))
 (segment (start 119.223028 108.99427) (end 114.991288 113.22601) (width 0.25) (layer F.Cu) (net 6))
 (segment (start 117.348 103.204) (end 117.598 103.204) (width 0.25) (layer F.Cu) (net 6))
 (segment (start 119.223028 104.829028) (end 119.223028 108.99427) (width 0.25) (layer F.Cu) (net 6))
 (segment (start 112.57999 113.22601) (end 110.49 115.316) (width 0.25) (layer F.Cu) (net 6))
 (segment (start 117.598 103.204) (end 119.223028 104.829028) (width 0.25) (layer F.Cu) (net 6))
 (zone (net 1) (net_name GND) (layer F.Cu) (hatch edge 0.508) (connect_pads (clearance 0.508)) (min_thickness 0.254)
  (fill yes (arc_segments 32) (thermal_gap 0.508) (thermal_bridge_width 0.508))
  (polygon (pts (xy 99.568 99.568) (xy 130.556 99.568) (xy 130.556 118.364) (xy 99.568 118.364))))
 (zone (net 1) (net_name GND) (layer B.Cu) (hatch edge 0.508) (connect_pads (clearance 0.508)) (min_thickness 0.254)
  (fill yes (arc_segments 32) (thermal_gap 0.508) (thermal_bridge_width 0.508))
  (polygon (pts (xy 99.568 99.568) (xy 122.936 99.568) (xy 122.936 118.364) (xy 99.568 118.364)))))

